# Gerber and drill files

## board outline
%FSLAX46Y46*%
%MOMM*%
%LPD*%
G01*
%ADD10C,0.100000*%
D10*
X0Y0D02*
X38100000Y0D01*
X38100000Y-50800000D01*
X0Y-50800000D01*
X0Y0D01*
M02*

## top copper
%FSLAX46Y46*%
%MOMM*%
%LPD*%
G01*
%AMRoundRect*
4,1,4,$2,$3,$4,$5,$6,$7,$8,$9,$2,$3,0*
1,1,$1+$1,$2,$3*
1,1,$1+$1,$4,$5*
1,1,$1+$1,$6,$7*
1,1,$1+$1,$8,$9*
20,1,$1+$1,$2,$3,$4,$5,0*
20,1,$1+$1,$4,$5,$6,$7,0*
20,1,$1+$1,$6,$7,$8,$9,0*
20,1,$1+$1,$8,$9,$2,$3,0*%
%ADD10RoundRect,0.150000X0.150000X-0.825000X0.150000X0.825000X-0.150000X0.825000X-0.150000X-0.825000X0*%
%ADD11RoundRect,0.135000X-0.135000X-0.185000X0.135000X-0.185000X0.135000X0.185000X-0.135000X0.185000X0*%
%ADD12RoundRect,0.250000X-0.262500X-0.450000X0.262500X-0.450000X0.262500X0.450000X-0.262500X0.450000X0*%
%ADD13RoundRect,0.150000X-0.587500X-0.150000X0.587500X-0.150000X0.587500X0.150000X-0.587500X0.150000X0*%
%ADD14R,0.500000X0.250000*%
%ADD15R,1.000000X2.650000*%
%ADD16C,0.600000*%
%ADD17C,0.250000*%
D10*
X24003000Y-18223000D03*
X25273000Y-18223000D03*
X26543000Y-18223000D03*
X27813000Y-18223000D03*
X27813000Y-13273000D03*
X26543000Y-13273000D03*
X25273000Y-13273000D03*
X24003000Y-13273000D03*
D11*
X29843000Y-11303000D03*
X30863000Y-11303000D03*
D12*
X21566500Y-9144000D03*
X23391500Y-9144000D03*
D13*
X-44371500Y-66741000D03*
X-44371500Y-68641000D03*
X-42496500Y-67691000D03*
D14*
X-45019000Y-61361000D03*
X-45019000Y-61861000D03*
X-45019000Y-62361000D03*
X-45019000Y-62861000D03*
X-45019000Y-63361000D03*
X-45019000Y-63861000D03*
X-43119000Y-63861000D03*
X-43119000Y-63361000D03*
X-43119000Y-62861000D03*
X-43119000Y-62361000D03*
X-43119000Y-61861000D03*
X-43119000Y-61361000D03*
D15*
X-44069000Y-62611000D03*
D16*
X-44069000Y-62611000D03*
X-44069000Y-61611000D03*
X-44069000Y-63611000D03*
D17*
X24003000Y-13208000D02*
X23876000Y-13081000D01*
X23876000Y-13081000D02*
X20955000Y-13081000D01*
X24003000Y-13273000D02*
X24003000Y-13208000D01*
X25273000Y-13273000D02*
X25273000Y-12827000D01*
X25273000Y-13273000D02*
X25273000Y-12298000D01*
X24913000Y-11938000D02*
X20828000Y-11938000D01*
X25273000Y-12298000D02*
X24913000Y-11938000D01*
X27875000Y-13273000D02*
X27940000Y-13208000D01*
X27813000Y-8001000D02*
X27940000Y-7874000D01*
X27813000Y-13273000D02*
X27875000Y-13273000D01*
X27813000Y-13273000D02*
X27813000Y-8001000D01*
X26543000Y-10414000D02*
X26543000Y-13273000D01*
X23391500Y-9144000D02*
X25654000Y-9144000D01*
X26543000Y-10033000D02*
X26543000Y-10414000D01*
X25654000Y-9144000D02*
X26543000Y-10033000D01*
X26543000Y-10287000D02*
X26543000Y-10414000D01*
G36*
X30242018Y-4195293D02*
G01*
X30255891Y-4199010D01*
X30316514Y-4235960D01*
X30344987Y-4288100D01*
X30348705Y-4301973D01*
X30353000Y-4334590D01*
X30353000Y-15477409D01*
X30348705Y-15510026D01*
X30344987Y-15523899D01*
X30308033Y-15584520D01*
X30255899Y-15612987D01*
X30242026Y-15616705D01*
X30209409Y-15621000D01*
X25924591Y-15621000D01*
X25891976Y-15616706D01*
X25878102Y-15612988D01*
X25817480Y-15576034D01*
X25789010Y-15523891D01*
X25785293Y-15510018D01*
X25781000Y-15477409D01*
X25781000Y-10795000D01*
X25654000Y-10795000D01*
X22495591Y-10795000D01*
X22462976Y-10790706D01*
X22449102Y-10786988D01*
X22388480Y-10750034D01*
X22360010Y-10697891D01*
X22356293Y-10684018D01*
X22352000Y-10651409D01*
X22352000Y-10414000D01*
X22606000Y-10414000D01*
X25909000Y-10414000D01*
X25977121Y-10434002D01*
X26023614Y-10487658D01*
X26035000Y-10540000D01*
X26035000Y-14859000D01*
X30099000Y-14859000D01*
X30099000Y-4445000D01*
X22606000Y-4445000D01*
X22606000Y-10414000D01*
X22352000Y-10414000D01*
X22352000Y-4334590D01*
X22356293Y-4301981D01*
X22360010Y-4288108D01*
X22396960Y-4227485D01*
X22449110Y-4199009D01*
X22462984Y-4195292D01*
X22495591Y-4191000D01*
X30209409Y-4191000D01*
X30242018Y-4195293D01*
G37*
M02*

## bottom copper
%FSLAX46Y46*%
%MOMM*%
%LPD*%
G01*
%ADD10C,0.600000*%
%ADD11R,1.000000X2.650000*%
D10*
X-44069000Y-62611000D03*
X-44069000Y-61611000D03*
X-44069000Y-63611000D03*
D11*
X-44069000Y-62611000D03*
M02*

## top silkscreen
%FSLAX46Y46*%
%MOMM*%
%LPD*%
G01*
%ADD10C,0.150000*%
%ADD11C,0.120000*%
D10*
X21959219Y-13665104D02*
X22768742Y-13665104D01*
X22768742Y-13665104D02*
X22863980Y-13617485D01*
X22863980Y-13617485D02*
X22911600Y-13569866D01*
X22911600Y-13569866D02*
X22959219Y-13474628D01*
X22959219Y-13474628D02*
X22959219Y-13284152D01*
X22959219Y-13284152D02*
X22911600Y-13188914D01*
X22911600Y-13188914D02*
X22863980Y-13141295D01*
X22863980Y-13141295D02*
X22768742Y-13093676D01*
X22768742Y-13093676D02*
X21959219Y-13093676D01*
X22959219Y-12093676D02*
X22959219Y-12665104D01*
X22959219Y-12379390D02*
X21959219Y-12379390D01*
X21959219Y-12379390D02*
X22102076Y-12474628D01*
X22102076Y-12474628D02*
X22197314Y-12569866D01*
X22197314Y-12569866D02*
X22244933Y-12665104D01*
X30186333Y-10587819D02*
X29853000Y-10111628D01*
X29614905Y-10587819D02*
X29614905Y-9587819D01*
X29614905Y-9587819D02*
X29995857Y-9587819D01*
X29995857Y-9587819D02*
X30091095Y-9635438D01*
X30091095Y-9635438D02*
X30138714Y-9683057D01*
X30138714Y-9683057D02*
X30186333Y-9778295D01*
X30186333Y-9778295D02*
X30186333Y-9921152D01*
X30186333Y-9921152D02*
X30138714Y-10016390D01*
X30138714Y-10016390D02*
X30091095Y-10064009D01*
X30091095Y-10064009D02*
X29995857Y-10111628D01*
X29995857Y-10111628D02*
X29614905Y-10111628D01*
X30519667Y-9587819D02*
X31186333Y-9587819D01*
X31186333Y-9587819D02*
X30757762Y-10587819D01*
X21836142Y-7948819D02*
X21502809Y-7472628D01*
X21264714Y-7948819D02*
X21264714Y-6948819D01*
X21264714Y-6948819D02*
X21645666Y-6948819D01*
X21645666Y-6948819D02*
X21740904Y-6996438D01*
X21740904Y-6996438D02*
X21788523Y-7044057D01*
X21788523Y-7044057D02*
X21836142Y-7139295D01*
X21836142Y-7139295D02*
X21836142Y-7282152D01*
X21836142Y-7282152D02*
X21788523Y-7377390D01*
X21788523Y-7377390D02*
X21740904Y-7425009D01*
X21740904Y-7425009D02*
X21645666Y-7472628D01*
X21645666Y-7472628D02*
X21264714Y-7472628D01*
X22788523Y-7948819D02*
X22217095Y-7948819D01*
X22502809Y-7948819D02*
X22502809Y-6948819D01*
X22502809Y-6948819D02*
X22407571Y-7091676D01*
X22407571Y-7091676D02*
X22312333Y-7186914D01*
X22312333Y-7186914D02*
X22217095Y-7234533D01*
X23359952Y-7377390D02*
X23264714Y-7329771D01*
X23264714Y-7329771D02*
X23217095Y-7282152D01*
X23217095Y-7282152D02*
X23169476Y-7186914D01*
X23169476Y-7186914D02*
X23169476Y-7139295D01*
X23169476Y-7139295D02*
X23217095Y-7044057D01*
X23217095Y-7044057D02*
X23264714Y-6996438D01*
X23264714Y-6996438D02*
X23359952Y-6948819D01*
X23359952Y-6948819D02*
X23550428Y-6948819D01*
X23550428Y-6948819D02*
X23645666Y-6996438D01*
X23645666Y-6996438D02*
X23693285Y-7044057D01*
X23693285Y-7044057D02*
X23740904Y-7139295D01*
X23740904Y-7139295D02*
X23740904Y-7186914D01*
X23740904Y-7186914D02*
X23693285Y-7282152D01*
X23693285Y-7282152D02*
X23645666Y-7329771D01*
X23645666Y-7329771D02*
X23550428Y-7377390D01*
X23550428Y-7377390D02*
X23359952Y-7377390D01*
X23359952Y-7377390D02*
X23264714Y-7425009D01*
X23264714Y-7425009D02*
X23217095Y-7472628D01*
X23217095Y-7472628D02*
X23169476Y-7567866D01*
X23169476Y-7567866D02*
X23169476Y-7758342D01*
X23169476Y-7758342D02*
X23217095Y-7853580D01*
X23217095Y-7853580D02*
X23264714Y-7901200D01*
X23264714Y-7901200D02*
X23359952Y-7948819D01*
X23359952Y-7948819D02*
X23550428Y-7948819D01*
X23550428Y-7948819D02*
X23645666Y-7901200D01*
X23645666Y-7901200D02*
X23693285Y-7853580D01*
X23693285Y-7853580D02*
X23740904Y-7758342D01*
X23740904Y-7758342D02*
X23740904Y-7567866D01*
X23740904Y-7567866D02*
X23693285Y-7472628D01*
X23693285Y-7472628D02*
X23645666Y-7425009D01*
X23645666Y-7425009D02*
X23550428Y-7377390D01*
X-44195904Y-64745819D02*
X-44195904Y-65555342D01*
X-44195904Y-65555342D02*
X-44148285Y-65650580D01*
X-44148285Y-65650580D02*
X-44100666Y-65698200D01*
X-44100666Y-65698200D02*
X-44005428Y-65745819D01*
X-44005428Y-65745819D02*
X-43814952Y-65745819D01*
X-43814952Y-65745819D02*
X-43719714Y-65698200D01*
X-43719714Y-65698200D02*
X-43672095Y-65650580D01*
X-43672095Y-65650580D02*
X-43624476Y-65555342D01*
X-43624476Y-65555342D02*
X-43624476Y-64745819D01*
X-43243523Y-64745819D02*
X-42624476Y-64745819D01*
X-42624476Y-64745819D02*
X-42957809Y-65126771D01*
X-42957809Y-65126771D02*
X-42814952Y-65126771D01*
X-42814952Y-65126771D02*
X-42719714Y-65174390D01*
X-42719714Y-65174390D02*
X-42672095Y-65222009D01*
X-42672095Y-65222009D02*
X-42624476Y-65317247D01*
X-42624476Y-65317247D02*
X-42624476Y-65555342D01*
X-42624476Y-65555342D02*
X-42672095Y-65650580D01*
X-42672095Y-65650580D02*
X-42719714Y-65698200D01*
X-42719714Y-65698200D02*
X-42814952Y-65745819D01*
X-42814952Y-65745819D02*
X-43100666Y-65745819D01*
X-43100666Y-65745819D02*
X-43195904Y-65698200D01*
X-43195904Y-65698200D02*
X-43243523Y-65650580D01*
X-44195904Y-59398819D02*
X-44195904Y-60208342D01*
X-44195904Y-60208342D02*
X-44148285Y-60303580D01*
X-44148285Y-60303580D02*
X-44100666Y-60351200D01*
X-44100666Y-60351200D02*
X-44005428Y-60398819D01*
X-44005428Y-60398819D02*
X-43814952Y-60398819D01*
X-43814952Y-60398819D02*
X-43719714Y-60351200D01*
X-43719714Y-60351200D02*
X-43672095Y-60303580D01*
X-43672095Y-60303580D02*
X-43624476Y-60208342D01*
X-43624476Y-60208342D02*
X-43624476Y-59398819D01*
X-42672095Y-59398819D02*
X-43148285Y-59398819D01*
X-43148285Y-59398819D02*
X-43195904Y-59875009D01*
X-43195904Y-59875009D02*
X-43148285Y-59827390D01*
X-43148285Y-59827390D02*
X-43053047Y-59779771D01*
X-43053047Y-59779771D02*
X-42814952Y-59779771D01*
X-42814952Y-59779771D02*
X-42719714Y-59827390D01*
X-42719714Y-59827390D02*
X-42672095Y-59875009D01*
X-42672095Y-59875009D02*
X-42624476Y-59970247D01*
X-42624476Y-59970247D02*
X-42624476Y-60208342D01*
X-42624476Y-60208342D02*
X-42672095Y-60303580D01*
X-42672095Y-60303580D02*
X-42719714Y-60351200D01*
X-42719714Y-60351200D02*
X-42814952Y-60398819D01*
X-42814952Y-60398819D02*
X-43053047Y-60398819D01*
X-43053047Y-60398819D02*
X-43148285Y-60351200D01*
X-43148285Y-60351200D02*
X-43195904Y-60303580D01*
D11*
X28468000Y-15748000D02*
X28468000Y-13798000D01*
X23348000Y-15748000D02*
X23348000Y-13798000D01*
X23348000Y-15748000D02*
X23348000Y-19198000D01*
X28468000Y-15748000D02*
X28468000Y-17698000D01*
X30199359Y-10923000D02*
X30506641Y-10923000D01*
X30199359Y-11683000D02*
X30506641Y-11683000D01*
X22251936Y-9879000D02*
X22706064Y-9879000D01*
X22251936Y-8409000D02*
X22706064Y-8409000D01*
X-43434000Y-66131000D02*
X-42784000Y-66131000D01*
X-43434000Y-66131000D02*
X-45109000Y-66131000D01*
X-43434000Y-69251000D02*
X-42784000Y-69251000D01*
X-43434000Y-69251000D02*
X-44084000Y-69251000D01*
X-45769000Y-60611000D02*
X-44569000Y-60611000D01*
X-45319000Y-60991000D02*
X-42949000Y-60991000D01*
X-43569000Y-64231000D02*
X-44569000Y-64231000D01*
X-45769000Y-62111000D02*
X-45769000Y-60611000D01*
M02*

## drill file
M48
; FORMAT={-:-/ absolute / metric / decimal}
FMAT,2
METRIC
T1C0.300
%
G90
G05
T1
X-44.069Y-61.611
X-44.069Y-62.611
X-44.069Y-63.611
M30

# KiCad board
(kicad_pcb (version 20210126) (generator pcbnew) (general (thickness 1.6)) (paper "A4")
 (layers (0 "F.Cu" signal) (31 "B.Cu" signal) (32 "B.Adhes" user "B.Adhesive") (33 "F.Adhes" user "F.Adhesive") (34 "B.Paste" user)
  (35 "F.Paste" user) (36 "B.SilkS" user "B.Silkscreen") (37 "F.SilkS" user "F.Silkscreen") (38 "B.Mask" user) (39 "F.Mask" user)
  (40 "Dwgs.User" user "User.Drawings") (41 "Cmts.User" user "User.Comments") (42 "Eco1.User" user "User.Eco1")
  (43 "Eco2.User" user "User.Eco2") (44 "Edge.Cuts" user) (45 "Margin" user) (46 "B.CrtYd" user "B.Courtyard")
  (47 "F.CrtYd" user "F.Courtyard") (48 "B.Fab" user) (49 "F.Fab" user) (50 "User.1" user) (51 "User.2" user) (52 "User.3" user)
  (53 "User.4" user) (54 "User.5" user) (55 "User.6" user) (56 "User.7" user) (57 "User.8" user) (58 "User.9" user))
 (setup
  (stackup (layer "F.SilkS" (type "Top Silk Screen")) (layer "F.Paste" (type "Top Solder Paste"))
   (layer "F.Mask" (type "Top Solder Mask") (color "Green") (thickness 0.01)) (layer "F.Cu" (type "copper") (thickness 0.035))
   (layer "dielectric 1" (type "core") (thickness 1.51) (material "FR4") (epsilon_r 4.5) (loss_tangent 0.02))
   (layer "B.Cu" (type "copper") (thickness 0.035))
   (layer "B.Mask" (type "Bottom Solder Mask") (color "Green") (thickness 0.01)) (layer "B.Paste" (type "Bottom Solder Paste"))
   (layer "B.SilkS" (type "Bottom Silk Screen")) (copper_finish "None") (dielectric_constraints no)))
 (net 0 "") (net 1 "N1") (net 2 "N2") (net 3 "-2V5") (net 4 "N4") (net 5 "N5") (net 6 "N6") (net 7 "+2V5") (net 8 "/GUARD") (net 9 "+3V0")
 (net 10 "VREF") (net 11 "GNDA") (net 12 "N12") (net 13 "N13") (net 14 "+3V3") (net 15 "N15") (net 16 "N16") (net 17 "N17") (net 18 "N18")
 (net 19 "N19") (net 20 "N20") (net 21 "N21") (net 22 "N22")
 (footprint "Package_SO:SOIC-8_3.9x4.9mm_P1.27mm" (layer "F.Cu") (at 25.908 15.748 90)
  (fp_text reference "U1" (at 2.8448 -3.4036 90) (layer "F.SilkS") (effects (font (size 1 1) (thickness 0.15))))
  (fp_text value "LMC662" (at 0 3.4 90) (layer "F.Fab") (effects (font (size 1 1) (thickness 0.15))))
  (fp_line (start 0 2.56) (end 1.95 2.56) (layer "F.SilkS") (width 0.12))
  (fp_line (start 0 -2.56) (end 1.95 -2.56) (layer "F.SilkS") (width 0.12))
  (fp_line (start 0 -2.56) (end -3.45 -2.56) (layer "F.SilkS") (width 0.12))
  (fp_line (start 0 2.56) (end -1.95 2.56) (layer "F.SilkS") (width 0.12))
  (pad "1" smd roundrect (at -2.475 -1.905 90) (locked) (size 1.95 0.6) (layers "F.Cu" "F.Paste" "F.Mask") (roundrect_rratio 0.25)
   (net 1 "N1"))
  (pad "2" smd roundrect (at -2.475 -0.635 90) (locked) (size 1.95 0.6) (layers "F.Cu" "F.Paste" "F.Mask") (roundrect_rratio 0.25)
   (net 1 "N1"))
  (pad "3" smd roundrect (at -2.475 0.635 90) (locked) (size 1.95 0.6) (layers "F.Cu" "F.Paste" "F.Mask") (roundrect_rratio 0.25)
   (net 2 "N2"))
  (pad "4" smd roundrect (at -2.475 1.905 90) (locked) (size 1.95 0.6) (layers "F.Cu" "F.Paste" "F.Mask") (roundrect_rratio 0.25)
   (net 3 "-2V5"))
  (pad "5" smd roundrect (at 2.475 1.905 90) (locked) (size 1.95 0.6) (layers "F.Cu" "F.Paste" "F.Mask") (roundrect_rratio 0.25)
   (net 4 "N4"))
  (pad "6" smd roundrect (at 2.475 0.635 90) (locked) (size 1.95 0.6) (layers "F.Cu" "F.Paste" "F.Mask") (roundrect_rratio 0.25)
   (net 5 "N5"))
  (pad "7" smd roundrect (at 2.475 -0.635 90) (locked) (size 1.95 0.6) (layers "F.Cu" "F.Paste" "F.Mask") (roundrect_rratio 0.25)
   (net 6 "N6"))
  (pad "8" smd roundrect (at 2.475 -1.905 90) (locked) (size 1.95 0.6) (layers "F.Cu" "F.Paste" "F.Mask") (roundrect_rratio 0.25)
   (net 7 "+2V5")))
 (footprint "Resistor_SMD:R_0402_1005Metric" (layer "F.Cu") (at 30.353 11.303)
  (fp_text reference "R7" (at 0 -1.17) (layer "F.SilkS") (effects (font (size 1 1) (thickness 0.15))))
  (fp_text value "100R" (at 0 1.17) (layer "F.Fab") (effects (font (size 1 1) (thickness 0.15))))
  (fp_line (start -0.153641 -0.38) (end 0.153641 -0.38) (layer "F.SilkS") (width 0.12))
  (fp_line (start -0.153641 0.38) (end 0.153641 0.38) (layer "F.SilkS") (width 0.12))
  (pad "1" smd roundrect (at -0.51 0) (locked) (size 0.54 0.64) (layers "F.Cu" "F.Paste" "F.Mask") (roundrect_rratio 0.25) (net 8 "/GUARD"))
  (pad "2" smd roundrect (at 0.51 0) (locked) (size 0.54 0.64) (layers "F.Cu" "F.Paste" "F.Mask") (roundrect_rratio 0.25) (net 1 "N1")))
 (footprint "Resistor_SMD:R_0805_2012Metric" (layer "F.Cu") (at 22.479 9.144)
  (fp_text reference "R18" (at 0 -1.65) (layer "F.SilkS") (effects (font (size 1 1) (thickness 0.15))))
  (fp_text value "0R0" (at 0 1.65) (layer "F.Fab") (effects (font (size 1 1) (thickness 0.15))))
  (fp_line (start -0.227064 0.735) (end 0.227064 0.735) (layer "F.SilkS") (width 0.12))
  (fp_line (start -0.227064 -0.735) (end 0.227064 -0.735) (layer "F.SilkS") (width 0.12))
  (pad "1" smd roundrect (at -0.9125 0) (locked) (size 1.025 1.4) (layers "F.Cu" "F.Paste" "F.Mask") (roundrect_rratio 0.243902)
   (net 2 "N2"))
  (pad "2" smd roundrect (at 0.9125 0) (locked) (size 1.025 1.4) (layers "F.Cu" "F.Paste" "F.Mask") (roundrect_rratio 0.243902) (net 5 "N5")))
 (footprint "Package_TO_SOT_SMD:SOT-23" (layer "F.Cu") (at -43.434 67.691)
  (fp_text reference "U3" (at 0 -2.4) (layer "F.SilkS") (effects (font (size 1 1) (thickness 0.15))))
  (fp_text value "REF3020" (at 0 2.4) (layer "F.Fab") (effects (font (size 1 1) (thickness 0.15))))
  (fp_line (start 0 -1.56) (end 0.65 -1.56) (layer "F.SilkS") (width 0.12))
  (fp_line (start 0 -1.56) (end -1.675 -1.56) (layer "F.SilkS") (width 0.12))
  (fp_line (start 0 1.56) (end 0.65 1.56) (layer "F.SilkS") (width 0.12))
  (fp_line (start 0 1.56) (end -0.65 1.56) (layer "F.SilkS") (width 0.12))
  (pad "1" smd roundrect (at -0.9375 -0.95) (locked) (size 1.475 0.6) (layers "F.Cu" "F.Paste" "F.Mask") (roundrect_rratio 0.25)
   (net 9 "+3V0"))
  (pad "2" smd roundrect (at -0.9375 0.95) (locked) (size 1.475 0.6) (layers "F.Cu" "F.Paste" "F.Mask") (roundrect_rratio 0.25)
   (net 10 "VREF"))
  (pad "3" smd roundrect (at 0.9375 0) (locked) (size 1.475 0.6) (layers "F.Cu" "F.Paste" "F.Mask") (roundrect_rratio 0.25) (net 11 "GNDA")))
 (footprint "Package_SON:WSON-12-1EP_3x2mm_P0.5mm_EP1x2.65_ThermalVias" (layer "F.Cu") (at -44.069 62.611)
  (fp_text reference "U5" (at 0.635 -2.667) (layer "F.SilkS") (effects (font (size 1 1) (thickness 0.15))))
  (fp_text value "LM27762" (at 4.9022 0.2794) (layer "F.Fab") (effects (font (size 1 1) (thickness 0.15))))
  (fp_line (start -1.7 -2) (end -0.5 -2) (layer "F.SilkS") (width 0.12))
  (fp_line (start -1.25 -1.62) (end 1.12 -1.62) (layer "F.SilkS") (width 0.12))
  (fp_line (start 0.5 1.62) (end -0.5 1.62) (layer "F.SilkS") (width 0.12))
  (fp_line (start -1.7 -0.5) (end -1.7 -2) (layer "F.SilkS") (width 0.12))
  (pad "" smd rect (at 0 0.5) (locked) (size 0.95 0.8) (layers "F.Paste"))
  (pad "" smd rect (at 0 -0.5) (locked) (size 0.95 0.8) (layers "F.Paste"))
  (pad "1" smd rect (at -0.95 -1.25) (locked) (size 0.5 0.25) (layers "F.Cu" "F.Paste" "F.Mask") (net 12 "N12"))
  (pad "2" smd rect (at -0.95 -0.75) (locked) (size 0.5 0.25) (layers "F.Cu" "F.Paste" "F.Mask") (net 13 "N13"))
  (pad "3" smd rect (at -0.95 -0.25) (locked) (size 0.5 0.25) (layers "F.Cu" "F.Paste" "F.Mask") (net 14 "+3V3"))
  (pad "4" smd rect (at -0.95 0.25) (locked) (size 0.5 0.25) (layers "F.Cu" "F.Paste" "F.Mask") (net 11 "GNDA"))
  (pad "5" smd rect (at -0.95 0.75) (locked) (size 0.5 0.25) (layers "F.Cu" "F.Paste" "F.Mask") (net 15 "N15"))
  (pad "6" smd rect (at -0.95 1.25) (locked) (size 0.5 0.25) (layers "F.Cu" "F.Paste" "F.Mask") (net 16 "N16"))
  (pad "7" smd rect (at 0.95 1.25) (locked) (size 0.5 0.25) (layers "F.Cu" "F.Paste" "F.Mask") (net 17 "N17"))
  (pad "8" smd rect (at 0.95 0.75) (locked) (size 0.5 0.25) (layers "F.Cu" "F.Paste" "F.Mask") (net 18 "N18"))
  (pad "9" smd rect (at 0.95 0.25) (locked) (size 0.5 0.25) (layers "F.Cu" "F.Paste" "F.Mask") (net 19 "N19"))
  (pad "10" smd rect (at 0.95 -0.25) (locked) (size 0.5 0.25) (layers "F.Cu" "F.Paste" "F.Mask") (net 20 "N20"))
  (pad "11" smd rect (at 0.95 -0.75) (locked) (size 0.5 0.25) (layers "F.Cu" "F.Paste" "F.Mask") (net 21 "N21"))
  (pad "12" smd rect (at 0.95 -1.25) (locked) (size 0.5 0.25) (layers "F.Cu" "F.Paste" "F.Mask") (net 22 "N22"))
  (pad "13" smd rect (at 0 0) (locked) (size 1 2.65) (layers "F.Cu" "F.Mask") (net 11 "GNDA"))
  (pad "13" thru_hole circle (at 0 0) (locked) (size 0.6 0.6) (drill 0.3) (layers *.Cu) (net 11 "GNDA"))
  (pad "13" thru_hole circle (at 0 -1 90) (locked) (size 0.6 0.6) (drill 0.3) (layers *.Cu) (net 11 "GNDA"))
  (pad "13" thru_hole circle (at 0 1) (locked) (size 0.6 0.6) (drill 0.3) (layers *.Cu) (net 11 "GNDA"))
  (pad "13" smd rect (at 0 0) (locked) (size 1 2.65) (layers "B.Cu") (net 11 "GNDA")))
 (gr_rect (start 0 0) (end 38.1 50.8) (layer "Edge.Cuts") (width 0.1) (fill none))
 (segment (start 24.003 13.208) (end 23.876 13.081) (width 0.25) (layer "F.Cu") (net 7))
 (segment (start 23.876 13.081) (end 20.955 13.081) (width 0.25) (layer "F.Cu") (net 7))
 (segment (start 24.003 13.273) (end 24.003 13.208) (width 0.25) (layer "F.Cu") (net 7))
 (segment (start 25.273 13.273) (end 25.273 12.827) (width 0.25) (layer "F.Cu") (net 6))
 (segment (start 25.273 13.273) (end 25.273 12.298) (width 0.25) (layer "F.Cu") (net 6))
 (segment (start 24.913 11.938) (end 20.828 11.938) (width 0.25) (layer "F.Cu") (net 6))
 (segment (start 25.273 12.298) (end 24.913 11.938) (width 0.25) (layer "F.Cu") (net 6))
 (segment (start 27.875 13.273) (end 27.94 13.208) (width 0.25) (layer "F.Cu") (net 4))
 (segment (start 27.813 8.001) (end 27.94 7.874) (width 0.25) (layer "F.Cu") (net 4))
 (segment (start 27.813 13.273) (end 27.875 13.273) (width 0.25) (layer "F.Cu") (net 4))
 (segment (start 27.813 13.273) (end 27.813 8.001) (width 0.25) (layer "F.Cu") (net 4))
 (segment (start 26.543 10.414) (end 26.543 13.273) (width 0.25) (layer "F.Cu") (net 5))
 (segment (start 23.3915 9.144) (end 25.654 9.144) (width 0.25) (layer "F.Cu") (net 5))
 (segment (start 26.543 10.033) (end 26.543 10.414) (width 0.25) (layer "F.Cu") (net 5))
 (segment (start 25.654 9.144) (end 26.543 10.033) (width 0.25) (layer "F.Cu") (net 5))
 (segment (start 26.543 10.287) (end 26.543 10.414) (width 0.25) (layer "F.Cu") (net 5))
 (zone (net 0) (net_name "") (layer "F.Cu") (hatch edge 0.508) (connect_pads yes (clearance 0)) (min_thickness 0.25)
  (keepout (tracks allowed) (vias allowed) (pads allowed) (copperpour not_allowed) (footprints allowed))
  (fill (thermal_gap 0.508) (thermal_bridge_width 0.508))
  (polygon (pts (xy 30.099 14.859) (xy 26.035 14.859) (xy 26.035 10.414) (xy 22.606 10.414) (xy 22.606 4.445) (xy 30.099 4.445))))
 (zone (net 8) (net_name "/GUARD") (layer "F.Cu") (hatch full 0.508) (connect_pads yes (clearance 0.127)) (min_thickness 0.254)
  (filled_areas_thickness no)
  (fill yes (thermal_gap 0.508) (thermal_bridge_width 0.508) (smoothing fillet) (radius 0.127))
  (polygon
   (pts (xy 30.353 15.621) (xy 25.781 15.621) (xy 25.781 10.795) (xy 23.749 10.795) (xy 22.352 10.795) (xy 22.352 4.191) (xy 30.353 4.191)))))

